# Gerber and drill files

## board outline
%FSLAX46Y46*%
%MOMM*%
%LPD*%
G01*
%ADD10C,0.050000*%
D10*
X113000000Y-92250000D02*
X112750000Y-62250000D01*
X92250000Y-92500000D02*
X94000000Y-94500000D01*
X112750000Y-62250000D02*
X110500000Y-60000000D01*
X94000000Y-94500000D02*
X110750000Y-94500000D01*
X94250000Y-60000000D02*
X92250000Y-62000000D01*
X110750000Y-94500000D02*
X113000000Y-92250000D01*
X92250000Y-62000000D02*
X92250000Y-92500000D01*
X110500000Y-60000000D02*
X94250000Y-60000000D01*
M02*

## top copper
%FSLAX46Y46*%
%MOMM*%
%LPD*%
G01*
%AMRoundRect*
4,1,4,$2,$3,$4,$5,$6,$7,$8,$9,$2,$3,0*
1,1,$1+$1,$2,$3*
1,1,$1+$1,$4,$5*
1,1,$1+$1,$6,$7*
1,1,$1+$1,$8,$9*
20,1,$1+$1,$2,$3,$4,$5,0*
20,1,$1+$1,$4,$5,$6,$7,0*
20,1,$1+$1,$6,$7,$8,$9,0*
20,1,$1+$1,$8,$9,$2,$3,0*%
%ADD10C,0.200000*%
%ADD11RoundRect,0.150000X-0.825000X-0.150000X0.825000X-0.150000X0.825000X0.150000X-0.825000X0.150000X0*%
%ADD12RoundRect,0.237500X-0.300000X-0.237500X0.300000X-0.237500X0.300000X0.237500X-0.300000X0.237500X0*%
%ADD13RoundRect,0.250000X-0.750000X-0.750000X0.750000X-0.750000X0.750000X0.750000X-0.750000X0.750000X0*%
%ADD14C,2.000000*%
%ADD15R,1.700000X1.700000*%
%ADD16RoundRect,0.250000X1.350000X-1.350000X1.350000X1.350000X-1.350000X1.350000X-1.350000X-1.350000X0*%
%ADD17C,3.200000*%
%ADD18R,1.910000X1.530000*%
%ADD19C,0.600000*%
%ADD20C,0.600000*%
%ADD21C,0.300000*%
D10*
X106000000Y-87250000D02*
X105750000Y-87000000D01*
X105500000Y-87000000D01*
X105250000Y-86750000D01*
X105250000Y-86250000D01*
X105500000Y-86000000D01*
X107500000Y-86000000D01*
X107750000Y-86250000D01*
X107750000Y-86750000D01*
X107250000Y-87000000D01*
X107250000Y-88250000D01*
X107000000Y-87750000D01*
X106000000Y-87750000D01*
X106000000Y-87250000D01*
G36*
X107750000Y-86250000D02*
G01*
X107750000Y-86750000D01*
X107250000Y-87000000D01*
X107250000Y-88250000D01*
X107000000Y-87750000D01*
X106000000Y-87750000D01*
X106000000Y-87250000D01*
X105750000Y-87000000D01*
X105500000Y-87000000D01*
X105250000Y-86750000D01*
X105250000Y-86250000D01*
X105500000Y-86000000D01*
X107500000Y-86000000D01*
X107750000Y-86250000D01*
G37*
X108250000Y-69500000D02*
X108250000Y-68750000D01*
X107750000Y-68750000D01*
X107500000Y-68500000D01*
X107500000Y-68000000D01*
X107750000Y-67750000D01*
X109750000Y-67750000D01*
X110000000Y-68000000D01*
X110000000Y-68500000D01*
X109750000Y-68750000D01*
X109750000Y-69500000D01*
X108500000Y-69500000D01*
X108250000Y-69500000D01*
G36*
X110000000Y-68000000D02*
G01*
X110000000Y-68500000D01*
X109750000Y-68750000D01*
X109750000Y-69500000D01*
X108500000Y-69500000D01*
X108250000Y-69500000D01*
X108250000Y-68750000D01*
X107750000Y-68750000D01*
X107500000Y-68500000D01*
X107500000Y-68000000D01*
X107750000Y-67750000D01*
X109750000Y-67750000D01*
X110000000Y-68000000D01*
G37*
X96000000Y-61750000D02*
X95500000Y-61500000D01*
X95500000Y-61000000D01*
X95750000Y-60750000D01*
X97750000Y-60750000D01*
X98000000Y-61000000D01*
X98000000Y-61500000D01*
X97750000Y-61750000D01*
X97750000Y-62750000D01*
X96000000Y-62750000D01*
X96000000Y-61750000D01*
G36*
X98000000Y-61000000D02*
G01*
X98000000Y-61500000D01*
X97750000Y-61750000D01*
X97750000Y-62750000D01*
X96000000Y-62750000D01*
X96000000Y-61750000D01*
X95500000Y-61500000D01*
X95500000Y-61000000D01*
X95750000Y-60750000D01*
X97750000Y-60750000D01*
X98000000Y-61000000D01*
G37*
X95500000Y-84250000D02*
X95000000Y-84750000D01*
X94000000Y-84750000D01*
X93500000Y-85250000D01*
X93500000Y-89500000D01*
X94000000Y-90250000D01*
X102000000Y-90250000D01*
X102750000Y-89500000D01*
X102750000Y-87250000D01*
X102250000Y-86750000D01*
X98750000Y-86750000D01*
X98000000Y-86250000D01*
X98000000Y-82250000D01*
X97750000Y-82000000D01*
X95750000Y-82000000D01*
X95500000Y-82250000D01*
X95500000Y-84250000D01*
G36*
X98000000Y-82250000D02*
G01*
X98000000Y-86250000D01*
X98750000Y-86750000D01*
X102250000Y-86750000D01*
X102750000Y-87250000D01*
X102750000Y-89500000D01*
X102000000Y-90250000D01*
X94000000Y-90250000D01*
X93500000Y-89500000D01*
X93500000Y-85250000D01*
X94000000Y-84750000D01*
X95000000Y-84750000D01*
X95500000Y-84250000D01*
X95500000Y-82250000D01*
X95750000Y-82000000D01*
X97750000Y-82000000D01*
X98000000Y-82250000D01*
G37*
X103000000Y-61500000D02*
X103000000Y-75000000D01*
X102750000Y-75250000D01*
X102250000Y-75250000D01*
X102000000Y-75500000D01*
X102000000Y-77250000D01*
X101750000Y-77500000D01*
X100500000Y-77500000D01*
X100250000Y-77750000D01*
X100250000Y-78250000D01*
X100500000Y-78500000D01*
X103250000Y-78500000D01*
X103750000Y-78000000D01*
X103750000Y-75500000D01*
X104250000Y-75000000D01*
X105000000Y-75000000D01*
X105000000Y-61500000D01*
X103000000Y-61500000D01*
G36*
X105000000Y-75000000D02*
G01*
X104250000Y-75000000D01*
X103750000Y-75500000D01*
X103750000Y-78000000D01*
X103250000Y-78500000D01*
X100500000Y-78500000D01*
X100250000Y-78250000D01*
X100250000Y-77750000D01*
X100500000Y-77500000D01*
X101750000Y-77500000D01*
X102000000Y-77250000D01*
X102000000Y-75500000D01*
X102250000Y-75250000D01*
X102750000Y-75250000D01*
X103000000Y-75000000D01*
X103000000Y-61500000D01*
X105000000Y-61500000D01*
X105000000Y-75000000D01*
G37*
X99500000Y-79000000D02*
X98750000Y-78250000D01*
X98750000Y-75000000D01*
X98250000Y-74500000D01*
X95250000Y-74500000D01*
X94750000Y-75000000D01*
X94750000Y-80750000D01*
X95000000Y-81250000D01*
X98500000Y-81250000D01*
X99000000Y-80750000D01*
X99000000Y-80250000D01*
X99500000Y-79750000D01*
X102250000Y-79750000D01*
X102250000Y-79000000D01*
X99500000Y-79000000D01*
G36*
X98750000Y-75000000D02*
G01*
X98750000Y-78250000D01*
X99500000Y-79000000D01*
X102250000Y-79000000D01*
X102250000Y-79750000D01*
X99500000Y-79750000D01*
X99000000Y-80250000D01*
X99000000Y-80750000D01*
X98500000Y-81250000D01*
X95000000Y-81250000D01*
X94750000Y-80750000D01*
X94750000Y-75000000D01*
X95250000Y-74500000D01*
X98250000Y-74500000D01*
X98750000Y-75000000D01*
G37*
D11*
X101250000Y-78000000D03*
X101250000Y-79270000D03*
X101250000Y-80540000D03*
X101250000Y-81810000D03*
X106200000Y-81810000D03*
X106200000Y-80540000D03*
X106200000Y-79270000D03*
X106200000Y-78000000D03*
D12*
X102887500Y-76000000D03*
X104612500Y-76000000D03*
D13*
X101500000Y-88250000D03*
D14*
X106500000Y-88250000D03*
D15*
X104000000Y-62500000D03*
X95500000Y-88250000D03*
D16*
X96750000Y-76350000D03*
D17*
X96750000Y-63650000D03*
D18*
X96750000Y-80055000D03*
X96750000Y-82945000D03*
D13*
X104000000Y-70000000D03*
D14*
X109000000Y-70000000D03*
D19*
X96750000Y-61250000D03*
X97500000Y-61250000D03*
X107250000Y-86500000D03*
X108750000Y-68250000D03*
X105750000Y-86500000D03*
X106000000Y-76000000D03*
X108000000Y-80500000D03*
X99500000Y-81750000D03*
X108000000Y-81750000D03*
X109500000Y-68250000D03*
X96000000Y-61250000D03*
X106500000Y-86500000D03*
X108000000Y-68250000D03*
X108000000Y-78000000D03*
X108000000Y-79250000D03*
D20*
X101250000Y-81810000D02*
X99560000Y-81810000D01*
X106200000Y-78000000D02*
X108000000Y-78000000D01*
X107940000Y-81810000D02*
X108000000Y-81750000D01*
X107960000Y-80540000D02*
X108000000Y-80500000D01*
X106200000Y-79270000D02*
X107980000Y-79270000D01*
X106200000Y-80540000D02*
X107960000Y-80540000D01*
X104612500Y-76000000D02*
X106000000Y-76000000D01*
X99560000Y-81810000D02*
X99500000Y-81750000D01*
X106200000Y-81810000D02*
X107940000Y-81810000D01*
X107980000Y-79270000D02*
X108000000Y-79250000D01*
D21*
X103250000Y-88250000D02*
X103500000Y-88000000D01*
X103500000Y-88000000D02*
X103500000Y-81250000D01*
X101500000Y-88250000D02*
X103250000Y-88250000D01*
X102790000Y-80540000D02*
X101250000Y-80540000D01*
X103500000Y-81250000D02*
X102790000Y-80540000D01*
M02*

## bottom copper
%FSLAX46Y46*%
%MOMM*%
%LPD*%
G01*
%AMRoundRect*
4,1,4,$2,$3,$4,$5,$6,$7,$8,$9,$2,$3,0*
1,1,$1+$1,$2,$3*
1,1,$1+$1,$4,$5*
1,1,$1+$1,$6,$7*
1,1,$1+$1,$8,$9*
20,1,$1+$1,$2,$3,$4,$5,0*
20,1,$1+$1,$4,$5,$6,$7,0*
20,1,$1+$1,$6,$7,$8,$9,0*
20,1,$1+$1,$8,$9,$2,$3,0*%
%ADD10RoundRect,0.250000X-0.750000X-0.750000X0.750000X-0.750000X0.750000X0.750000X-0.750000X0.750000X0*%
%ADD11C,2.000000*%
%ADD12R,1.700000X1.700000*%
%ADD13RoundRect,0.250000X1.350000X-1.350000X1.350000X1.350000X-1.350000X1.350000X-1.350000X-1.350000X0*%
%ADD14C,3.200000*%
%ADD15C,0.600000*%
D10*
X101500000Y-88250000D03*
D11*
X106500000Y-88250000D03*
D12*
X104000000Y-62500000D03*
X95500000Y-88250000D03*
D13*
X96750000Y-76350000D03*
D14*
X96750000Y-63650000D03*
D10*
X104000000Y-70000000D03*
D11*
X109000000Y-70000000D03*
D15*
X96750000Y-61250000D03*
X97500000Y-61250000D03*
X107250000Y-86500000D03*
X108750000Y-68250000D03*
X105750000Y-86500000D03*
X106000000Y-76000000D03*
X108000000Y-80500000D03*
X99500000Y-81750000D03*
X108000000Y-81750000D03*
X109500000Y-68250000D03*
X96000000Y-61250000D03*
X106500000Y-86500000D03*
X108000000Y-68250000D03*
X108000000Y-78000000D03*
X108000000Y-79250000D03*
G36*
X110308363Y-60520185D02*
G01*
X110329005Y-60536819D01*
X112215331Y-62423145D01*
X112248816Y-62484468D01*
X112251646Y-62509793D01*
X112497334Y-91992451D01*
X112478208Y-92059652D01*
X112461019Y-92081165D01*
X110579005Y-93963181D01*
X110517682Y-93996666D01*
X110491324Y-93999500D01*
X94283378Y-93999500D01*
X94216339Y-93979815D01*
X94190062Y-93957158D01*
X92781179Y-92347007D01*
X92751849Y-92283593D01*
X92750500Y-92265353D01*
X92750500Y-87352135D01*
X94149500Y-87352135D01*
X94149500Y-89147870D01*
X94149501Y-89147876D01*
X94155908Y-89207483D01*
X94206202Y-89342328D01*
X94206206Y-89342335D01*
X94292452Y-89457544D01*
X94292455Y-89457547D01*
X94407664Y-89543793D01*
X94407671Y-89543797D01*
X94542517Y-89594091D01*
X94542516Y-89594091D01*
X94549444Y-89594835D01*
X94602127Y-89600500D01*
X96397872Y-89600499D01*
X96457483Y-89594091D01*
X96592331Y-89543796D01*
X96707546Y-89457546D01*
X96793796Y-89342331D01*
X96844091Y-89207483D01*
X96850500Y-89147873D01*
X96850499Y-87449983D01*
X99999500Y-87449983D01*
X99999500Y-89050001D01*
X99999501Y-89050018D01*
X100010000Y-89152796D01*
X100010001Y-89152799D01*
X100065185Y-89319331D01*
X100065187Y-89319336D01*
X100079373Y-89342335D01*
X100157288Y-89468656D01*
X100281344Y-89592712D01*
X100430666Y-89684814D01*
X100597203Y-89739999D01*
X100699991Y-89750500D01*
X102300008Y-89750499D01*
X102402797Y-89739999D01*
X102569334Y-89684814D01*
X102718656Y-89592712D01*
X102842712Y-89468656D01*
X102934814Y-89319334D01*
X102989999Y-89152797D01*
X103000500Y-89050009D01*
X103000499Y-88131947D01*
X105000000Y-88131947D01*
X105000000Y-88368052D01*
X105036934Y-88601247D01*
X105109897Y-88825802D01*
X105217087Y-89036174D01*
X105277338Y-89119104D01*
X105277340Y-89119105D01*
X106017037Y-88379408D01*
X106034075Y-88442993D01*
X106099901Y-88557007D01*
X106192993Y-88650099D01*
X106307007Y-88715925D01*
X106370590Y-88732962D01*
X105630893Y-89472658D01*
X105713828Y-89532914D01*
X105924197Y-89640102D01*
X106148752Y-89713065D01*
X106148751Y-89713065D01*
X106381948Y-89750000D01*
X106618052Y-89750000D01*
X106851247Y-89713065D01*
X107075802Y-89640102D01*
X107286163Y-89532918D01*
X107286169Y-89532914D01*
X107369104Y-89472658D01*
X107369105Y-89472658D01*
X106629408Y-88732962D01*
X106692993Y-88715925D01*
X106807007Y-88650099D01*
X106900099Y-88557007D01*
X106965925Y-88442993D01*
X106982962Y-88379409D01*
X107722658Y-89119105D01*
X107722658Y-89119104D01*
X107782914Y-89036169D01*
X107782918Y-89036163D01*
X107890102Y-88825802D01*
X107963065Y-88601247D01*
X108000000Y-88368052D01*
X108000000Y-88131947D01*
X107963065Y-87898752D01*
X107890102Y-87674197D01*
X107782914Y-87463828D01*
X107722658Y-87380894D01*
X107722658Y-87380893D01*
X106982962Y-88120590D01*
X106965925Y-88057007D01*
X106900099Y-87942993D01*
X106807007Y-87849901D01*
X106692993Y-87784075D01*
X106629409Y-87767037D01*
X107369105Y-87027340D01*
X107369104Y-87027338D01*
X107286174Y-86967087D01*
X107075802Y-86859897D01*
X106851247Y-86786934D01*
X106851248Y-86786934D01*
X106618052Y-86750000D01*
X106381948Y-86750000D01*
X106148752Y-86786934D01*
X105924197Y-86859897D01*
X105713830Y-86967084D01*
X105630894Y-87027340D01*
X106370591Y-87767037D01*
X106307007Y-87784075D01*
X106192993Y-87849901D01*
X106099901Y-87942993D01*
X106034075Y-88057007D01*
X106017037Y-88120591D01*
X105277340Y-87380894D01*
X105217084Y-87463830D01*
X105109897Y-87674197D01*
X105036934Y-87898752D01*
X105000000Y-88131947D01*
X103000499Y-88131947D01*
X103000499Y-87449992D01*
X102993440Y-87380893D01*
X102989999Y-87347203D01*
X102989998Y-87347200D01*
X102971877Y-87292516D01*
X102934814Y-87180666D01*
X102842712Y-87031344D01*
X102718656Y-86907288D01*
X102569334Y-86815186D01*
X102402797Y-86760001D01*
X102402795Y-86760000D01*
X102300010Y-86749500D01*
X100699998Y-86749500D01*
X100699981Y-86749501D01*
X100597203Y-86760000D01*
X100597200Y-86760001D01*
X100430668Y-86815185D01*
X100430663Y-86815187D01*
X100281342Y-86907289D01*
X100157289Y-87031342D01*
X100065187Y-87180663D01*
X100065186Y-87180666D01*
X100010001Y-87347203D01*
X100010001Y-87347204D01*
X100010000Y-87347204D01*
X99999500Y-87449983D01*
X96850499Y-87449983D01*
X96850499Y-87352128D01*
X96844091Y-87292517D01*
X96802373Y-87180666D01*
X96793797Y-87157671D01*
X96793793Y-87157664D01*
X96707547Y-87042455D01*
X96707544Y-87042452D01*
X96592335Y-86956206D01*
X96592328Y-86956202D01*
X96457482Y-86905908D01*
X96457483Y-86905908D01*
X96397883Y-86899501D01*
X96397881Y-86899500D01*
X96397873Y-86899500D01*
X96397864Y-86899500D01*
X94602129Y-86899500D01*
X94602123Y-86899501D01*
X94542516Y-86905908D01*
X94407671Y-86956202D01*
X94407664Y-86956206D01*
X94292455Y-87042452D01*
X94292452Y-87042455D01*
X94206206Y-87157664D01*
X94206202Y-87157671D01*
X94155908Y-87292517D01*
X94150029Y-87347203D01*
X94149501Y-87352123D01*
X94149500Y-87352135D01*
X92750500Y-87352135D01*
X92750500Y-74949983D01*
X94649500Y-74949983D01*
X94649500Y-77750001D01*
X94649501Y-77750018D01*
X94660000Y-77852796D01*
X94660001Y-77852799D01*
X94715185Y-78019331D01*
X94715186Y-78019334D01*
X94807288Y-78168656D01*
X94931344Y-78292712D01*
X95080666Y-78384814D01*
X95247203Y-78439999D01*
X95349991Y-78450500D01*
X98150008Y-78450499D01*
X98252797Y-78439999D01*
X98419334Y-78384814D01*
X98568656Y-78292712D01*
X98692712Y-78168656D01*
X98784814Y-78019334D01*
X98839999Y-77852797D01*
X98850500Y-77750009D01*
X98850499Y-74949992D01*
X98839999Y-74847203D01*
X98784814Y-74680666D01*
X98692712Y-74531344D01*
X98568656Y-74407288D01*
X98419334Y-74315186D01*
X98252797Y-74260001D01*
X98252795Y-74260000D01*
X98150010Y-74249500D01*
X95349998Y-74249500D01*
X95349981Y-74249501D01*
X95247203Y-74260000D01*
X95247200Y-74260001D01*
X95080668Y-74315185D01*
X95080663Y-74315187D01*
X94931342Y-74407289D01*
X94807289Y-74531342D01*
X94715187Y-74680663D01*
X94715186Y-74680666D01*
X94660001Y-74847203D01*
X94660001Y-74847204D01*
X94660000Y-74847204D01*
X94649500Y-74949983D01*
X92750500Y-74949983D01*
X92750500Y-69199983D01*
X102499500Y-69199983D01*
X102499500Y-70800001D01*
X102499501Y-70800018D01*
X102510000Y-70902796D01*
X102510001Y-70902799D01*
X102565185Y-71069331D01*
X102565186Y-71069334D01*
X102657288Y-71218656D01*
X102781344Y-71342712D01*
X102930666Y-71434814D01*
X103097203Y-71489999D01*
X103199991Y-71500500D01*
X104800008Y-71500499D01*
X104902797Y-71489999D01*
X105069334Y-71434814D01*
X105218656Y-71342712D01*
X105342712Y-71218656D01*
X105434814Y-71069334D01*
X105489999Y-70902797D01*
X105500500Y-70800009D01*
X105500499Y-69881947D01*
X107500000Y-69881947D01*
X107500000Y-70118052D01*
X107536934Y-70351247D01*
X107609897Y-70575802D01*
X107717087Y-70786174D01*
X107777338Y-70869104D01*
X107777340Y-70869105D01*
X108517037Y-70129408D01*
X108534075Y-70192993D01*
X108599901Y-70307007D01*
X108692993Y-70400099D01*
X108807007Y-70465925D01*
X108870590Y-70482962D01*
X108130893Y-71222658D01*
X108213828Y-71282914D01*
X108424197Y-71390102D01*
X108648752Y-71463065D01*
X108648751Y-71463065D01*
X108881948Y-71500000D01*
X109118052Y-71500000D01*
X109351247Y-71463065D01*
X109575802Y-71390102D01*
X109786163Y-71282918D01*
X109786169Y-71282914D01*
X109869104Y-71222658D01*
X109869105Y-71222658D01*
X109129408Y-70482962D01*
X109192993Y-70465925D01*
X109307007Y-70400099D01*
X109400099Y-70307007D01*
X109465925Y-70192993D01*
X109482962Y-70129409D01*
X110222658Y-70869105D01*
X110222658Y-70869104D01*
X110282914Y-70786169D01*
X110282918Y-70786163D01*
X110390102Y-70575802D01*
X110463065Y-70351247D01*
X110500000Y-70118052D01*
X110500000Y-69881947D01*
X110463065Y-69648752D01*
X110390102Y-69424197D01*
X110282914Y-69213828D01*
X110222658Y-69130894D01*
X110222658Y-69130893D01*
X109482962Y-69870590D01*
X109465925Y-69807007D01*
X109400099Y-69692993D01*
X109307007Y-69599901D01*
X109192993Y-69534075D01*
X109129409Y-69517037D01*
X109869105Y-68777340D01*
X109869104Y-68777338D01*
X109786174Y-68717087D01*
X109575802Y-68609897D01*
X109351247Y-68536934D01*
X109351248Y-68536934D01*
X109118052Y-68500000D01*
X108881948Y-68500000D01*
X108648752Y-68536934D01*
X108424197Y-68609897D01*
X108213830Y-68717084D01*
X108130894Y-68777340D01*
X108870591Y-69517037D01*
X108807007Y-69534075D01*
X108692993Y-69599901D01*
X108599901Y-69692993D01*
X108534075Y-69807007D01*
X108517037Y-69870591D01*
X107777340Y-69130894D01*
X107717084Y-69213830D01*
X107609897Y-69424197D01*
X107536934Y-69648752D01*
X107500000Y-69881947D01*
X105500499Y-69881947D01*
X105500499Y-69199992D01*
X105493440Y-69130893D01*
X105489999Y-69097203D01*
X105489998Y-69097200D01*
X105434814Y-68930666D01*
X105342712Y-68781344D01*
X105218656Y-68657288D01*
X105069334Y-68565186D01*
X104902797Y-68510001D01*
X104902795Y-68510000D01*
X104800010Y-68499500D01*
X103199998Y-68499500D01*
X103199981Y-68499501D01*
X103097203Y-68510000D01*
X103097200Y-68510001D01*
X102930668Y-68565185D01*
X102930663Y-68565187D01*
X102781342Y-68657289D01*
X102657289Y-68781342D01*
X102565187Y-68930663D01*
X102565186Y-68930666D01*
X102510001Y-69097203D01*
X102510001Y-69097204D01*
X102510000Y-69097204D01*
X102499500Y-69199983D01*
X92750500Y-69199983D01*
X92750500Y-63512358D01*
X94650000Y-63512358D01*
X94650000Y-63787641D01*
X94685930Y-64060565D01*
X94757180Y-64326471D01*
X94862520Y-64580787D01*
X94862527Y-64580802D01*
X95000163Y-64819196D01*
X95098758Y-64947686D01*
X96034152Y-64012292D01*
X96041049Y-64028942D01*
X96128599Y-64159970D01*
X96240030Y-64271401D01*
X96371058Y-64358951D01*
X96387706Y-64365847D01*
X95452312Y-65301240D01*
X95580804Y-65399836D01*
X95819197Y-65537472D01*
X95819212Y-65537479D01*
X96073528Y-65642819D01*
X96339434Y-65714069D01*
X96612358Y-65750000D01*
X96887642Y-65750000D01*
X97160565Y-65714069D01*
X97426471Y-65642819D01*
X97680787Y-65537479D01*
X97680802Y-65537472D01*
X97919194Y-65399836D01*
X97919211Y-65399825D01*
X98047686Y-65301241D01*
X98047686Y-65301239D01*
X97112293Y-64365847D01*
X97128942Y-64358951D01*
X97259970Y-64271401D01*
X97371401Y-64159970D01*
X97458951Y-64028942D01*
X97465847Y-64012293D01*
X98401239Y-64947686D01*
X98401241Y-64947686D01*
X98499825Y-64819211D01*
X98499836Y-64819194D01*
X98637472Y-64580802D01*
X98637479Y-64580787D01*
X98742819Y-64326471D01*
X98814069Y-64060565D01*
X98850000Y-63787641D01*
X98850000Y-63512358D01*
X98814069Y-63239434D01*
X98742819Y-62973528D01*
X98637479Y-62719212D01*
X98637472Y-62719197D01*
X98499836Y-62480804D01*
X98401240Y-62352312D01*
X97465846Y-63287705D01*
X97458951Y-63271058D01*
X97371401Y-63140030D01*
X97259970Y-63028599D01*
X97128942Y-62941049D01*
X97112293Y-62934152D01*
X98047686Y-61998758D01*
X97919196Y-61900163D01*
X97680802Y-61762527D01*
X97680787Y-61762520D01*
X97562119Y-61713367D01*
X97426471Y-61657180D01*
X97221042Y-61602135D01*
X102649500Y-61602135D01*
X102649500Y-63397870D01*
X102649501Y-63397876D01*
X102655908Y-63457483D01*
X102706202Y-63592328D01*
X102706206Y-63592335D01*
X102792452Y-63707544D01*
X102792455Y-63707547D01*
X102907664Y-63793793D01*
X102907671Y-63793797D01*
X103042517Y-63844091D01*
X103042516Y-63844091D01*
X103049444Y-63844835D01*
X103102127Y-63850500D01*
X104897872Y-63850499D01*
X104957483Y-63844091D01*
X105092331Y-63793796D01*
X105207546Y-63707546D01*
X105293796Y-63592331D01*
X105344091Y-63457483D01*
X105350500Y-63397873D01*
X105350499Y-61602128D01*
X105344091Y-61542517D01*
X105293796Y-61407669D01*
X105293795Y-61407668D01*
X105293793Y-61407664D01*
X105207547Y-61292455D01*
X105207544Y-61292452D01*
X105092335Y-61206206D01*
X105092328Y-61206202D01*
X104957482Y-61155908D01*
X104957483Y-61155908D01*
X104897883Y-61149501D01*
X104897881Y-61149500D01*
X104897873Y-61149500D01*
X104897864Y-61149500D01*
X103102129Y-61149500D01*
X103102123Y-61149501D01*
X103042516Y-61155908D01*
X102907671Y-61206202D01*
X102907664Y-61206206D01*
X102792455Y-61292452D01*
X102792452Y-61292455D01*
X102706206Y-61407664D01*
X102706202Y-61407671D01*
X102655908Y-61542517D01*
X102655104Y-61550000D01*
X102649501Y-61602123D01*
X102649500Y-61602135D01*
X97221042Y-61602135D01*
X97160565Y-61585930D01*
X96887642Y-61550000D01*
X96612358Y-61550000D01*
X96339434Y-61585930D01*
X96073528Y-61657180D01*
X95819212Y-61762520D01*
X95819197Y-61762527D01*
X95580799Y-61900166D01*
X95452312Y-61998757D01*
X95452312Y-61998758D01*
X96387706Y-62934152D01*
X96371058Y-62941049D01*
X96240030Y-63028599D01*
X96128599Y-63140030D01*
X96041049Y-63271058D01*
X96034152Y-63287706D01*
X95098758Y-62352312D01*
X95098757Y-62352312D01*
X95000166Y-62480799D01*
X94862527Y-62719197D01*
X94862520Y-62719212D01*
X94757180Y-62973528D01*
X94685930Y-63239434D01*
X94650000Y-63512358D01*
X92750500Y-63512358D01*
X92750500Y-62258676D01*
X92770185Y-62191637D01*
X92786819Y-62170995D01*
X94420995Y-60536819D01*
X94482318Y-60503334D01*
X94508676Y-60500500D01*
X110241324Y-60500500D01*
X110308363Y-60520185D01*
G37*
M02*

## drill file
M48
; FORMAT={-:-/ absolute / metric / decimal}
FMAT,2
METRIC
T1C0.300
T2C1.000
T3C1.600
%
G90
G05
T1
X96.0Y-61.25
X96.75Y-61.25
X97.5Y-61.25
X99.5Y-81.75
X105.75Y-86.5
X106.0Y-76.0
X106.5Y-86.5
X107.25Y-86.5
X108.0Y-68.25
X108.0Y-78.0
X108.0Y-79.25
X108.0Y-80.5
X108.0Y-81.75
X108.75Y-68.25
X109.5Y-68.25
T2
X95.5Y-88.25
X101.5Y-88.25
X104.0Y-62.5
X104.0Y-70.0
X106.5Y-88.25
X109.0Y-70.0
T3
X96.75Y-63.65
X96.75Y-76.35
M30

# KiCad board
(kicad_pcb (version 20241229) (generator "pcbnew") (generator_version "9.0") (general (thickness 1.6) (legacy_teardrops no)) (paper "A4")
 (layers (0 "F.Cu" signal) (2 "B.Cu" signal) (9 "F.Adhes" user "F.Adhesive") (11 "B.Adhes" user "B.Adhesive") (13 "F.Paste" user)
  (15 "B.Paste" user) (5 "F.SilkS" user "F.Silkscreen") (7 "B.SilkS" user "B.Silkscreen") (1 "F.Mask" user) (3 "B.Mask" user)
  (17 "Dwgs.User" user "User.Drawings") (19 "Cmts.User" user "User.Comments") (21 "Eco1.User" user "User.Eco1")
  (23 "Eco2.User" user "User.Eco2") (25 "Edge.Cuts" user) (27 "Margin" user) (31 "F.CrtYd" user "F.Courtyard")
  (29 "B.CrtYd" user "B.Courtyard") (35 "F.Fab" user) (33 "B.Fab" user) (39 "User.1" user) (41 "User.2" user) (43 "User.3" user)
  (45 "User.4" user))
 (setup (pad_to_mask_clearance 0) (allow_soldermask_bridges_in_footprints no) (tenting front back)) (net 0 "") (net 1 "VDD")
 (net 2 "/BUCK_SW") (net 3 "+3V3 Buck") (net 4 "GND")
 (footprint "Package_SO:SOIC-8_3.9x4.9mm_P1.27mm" (layer "F.Cu") (at 103.725 79.905)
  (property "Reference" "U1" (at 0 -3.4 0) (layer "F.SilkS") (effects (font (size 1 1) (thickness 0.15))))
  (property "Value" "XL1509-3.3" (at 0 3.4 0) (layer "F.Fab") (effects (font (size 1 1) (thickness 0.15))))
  (pad "1" smd roundrect (at -2.475 -1.905) (size 1.95 0.6) (layers "F.Cu" "F.Mask" "F.Paste") (roundrect_rratio 0.25) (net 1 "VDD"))
  (pad "2" smd roundrect (at -2.475 -0.635) (size 1.95 0.6) (layers "F.Cu" "F.Mask" "F.Paste") (roundrect_rratio 0.25) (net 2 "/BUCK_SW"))
  (pad "3" smd roundrect (at -2.475 0.635) (size 1.95 0.6) (layers "F.Cu" "F.Mask" "F.Paste") (roundrect_rratio 0.25) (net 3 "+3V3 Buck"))
  (pad "4" smd roundrect (at -2.475 1.905) (size 1.95 0.6) (layers "F.Cu" "F.Mask" "F.Paste") (roundrect_rratio 0.25) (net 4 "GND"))
  (pad "5" smd roundrect (at 2.475 1.905) (size 1.95 0.6) (layers "F.Cu" "F.Mask" "F.Paste") (roundrect_rratio 0.25) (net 4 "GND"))
  (pad "6" smd roundrect (at 2.475 0.635) (size 1.95 0.6) (layers "F.Cu" "F.Mask" "F.Paste") (roundrect_rratio 0.25) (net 4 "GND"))
  (pad "7" smd roundrect (at 2.475 -0.635) (size 1.95 0.6) (layers "F.Cu" "F.Mask" "F.Paste") (roundrect_rratio 0.25) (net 4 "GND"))
  (pad "8" smd roundrect (at 2.475 -1.905) (size 1.95 0.6) (layers "F.Cu" "F.Mask" "F.Paste") (roundrect_rratio 0.25) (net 4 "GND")))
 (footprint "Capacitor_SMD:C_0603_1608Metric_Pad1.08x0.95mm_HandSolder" (layer "F.Cu") (at 103.75 76)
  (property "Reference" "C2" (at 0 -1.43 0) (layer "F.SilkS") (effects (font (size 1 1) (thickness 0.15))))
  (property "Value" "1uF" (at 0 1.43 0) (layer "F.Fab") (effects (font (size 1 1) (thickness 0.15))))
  (pad "1" smd roundrect (at -0.8625 0) (size 1.075 0.95) (layers "F.Cu" "F.Mask" "F.Paste") (roundrect_rratio 0.25) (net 1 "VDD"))
  (pad "2" smd roundrect (at 0.8625 0) (size 1.075 0.95) (layers "F.Cu" "F.Mask" "F.Paste") (roundrect_rratio 0.25) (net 4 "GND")))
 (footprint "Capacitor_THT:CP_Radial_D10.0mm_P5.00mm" (layer "F.Cu") (at 101.5 88.25)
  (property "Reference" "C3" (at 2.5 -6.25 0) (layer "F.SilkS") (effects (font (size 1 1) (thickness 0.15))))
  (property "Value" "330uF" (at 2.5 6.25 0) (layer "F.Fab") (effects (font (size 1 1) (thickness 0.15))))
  (pad "1" thru_hole roundrect (at 0 0) (size 2 2) (drill 1) (layers "*.Cu" "*.Mask") (remove_unused_layers no) (roundrect_rratio 0.125)
   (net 3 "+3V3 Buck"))
  (pad "2" thru_hole circle (at 5 0) (size 2 2) (drill 1) (layers "*.Cu" "*.Mask") (remove_unused_layers no) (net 4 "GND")))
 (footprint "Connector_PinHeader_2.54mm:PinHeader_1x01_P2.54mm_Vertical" (layer "F.Cu") (at 104 62.5)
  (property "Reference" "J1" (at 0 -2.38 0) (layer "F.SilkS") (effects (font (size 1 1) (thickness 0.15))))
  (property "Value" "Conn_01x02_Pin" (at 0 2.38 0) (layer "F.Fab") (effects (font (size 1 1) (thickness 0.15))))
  (pad "1" thru_hole rect (at 0 0) (size 1.7 1.7) (drill 1) (layers "*.Cu" "*.Mask") (remove_unused_layers no) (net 1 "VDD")))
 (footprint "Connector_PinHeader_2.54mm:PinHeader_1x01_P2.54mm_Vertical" (layer "F.Cu") (at 95.5 88.25)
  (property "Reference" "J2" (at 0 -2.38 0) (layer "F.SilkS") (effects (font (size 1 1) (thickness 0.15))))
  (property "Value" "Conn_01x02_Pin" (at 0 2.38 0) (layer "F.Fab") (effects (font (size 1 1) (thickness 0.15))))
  (pad "1" thru_hole rect (at 0 0) (size 1.7 1.7) (drill 1) (layers "*.Cu" "*.Mask") (remove_unused_layers no) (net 3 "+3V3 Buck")))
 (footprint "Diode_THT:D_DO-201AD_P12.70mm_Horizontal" (layer "F.Cu") (at 96.75 76.35 90)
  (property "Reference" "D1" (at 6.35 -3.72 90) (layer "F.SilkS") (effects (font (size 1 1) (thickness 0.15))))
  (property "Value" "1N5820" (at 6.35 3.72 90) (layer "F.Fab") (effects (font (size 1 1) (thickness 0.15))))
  (pad "1" thru_hole roundrect (at 0 0 90) (size 3.2 3.2) (drill 1.6) (layers "*.Cu" "*.Mask") (remove_unused_layers no)
   (roundrect_rratio 0.078125) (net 2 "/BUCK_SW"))
  (pad "2" thru_hole circle (at 12.7 0 90) (size 3.2 3.2) (drill 1.6) (layers "*.Cu" "*.Mask") (remove_unused_layers no) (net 4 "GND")))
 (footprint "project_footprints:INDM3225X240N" (layer "F.Cu") (at 96.75 81.5 -90)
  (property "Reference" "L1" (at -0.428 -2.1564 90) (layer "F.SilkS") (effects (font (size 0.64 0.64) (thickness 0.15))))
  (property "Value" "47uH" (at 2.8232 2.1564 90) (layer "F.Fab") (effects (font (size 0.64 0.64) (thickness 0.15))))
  (pad "1" smd rect (at -1.445 0 270) (size 1.53 1.91) (layers "F.Cu" "F.Mask" "F.Paste") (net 2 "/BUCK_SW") (solder_mask_margin 0.102))
  (pad "2" smd rect (at 1.445 0 270) (size 1.53 1.91) (layers "F.Cu" "F.Mask" "F.Paste") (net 3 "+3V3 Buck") (solder_mask_margin 0.102)))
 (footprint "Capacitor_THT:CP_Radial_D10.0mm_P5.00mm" (layer "F.Cu") (at 104 70)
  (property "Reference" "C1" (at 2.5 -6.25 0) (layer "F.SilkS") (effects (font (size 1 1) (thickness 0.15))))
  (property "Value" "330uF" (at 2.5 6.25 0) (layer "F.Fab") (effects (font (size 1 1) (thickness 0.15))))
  (pad "1" thru_hole roundrect (at 0 0) (size 2 2) (drill 1) (layers "*.Cu" "*.Mask") (remove_unused_layers no) (roundrect_rratio 0.125)
   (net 1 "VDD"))
  (pad "2" thru_hole circle (at 5 0) (size 2 2) (drill 1) (layers "*.Cu" "*.Mask") (remove_unused_layers no) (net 4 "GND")))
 (gr_poly
  (pts (xy 106 87.25) (xy 105.75 87) (xy 105.5 87) (xy 105.25 86.75) (xy 105.25 86.25) (xy 105.5 86) (xy 107.5 86) (xy 107.75 86.25)
   (xy 107.75 86.75) (xy 107.25 87) (xy 107.25 88.25) (xy 107.25 88.25) (xy 107 87.75) (xy 106 87.75))
  (stroke (width 0.2) (type solid)) (fill yes) (layer "F.Cu") (net 4))
 (gr_poly
  (pts (xy 108.25 69.5) (xy 108.25 68.75) (xy 107.75 68.75) (xy 107.5 68.5) (xy 107.5 68) (xy 107.75 67.75) (xy 109.75 67.75) (xy 110 68)
   (xy 110 68.5) (xy 109.75 68.75) (xy 109.75 69.5) (xy 108.5 69.5))
  (stroke (width 0.2) (type solid)) (fill yes) (layer "F.Cu") (net 4))
 (gr_poly
  (pts (xy 96 61.75) (xy 95.5 61.5) (xy 95.5 61) (xy 95.75 60.75) (xy 97.75 60.75) (xy 98 61) (xy 98 61.5) (xy 97.75 61.75) (xy 97.75 62.75)
   (xy 96 62.75))
  (stroke (width 0.2) (type solid)) (fill yes) (layer "F.Cu") (net 4))
 (gr_poly
  (pts (xy 95.5 84.25) (xy 95 84.75) (xy 94 84.75) (xy 93.5 85.25) (xy 93.5 89.5) (xy 94 90.25) (xy 102 90.25) (xy 102.75 89.5)
   (xy 102.75 87.25) (xy 102.25 86.75) (xy 98.75 86.75) (xy 98 86.25) (xy 98 82.25) (xy 97.75 82) (xy 95.75 82) (xy 95.5 82.25))
  (stroke (width 0.2) (type solid)) (fill yes) (layer "F.Cu") (net 3))
 (gr_poly
  (pts (xy 103 61.5) (xy 103 75) (xy 102.75 75.25) (xy 102.25 75.25) (xy 102 75.5) (xy 102 77.25) (xy 101.75 77.5) (xy 100.5 77.5)
   (xy 100.25 77.75) (xy 100.25 78.25) (xy 100.5 78.5) (xy 103.25 78.5) (xy 103.75 78) (xy 103.75 75.5) (xy 104.25 75) (xy 105 75)
   (xy 105 61.5))
  (stroke (width 0.2) (type solid)) (fill yes) (layer "F.Cu") (net 1))
 (gr_poly
  (pts (xy 99.5 79) (xy 98.75 78.25) (xy 98.75 75) (xy 98.25 74.5) (xy 95.25 74.5) (xy 94.75 75) (xy 94.75 80.75) (xy 95 81.25)
   (xy 98.5 81.25) (xy 99 80.75) (xy 99 80.25) (xy 99.5 79.75) (xy 102.25 79.75) (xy 102.25 79))
  (stroke (width 0.2) (type solid)) (fill yes) (layer "F.Cu") (net 2))
 (gr_line (start 113 92.25) (end 112.75 62.25) (stroke (width 0.05) (type default)) (layer "Edge.Cuts"))
 (gr_line (start 92.25 92.5) (end 94 94.5) (stroke (width 0.05) (type default)) (layer "Edge.Cuts"))
 (gr_line (start 112.75 62.25) (end 110.5 60) (stroke (width 0.05) (type default)) (layer "Edge.Cuts"))
 (gr_line (start 94 94.5) (end 110.75 94.5) (stroke (width 0.05) (type default)) (layer "Edge.Cuts"))
 (gr_line (start 94.25 60) (end 92.25 62) (stroke (width 0.05) (type default)) (layer "Edge.Cuts"))
 (gr_line (start 110.75 94.5) (end 113 92.25) (stroke (width 0.05) (type default)) (layer "Edge.Cuts"))
 (gr_line (start 92.25 62) (end 92.25 92.5) (stroke (width 0.05) (type default)) (layer "Edge.Cuts"))
 (gr_line (start 110.5 60) (end 94.25 60) (stroke (width 0.05) (type default)) (layer "Edge.Cuts"))
 (segment (start 101.25 81.81) (end 99.56 81.81) (width 0.6) (layer "F.Cu") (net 4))
 (segment (start 106.2 78) (end 108 78) (width 0.6) (layer "F.Cu") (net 4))
 (segment (start 107.94 81.81) (end 108 81.75) (width 0.6) (layer "F.Cu") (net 4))
 (segment (start 107.96 80.54) (end 108 80.5) (width 0.6) (layer "F.Cu") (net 4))
 (segment (start 106.2 79.27) (end 107.98 79.27) (width 0.6) (layer "F.Cu") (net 4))
 (segment (start 106.2 80.54) (end 107.96 80.54) (width 0.6) (layer "F.Cu") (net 4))
 (segment (start 104.6125 76) (end 106 76) (width 0.6) (layer "F.Cu") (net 4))
 (segment (start 99.56 81.81) (end 99.5 81.75) (width 0.6) (layer "F.Cu") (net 4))
 (segment (start 106.2 81.81) (end 107.94 81.81) (width 0.6) (layer "F.Cu") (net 4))
 (segment (start 107.98 79.27) (end 108 79.25) (width 0.6) (layer "F.Cu") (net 4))
 (via (at 96.75 61.25) (size 0.6) (drill 0.3) (layers "F.Cu" "B.Cu") (free yes) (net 4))
 (via (at 97.5 61.25) (size 0.6) (drill 0.3) (layers "F.Cu" "B.Cu") (free yes) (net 4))
 (via (at 107.25 86.5) (size 0.6) (drill 0.3) (layers "F.Cu" "B.Cu") (free yes) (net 4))
 (via (at 108.75 68.25) (size 0.6) (drill 0.3) (layers "F.Cu" "B.Cu") (free yes) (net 4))
 (via (at 105.75 86.5) (size 0.6) (drill 0.3) (layers "F.Cu" "B.Cu") (free yes) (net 4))
 (via (at 106 76) (size 0.6) (drill 0.3) (layers "F.Cu" "B.Cu") (free yes) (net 4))
 (via (at 108 80.5) (size 0.6) (drill 0.3) (layers "F.Cu" "B.Cu") (free yes) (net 4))
 (via (at 99.5 81.75) (size 0.6) (drill 0.3) (layers "F.Cu" "B.Cu") (free yes) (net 4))
 (via (at 108 81.75) (size 0.6) (drill 0.3) (layers "F.Cu" "B.Cu") (free yes) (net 4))
 (via (at 109.5 68.25) (size 0.6) (drill 0.3) (layers "F.Cu" "B.Cu") (free yes) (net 4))
 (via (at 96 61.25) (size 0.6) (drill 0.3) (layers "F.Cu" "B.Cu") (free yes) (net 4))
 (via (at 106.5 86.5) (size 0.6) (drill 0.3) (layers "F.Cu" "B.Cu") (free yes) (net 4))
 (via (at 108 68.25) (size 0.6) (drill 0.3) (layers "F.Cu" "B.Cu") (free yes) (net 4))
 (via (at 108 78) (size 0.6) (drill 0.3) (layers "F.Cu" "B.Cu") (free yes) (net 4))
 (via (at 108 79.25) (size 0.6) (drill 0.3) (layers "F.Cu" "B.Cu") (free yes) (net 4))
 (segment (start 103.25 88.25) (end 103.5 88) (width 0.3) (layer "F.Cu") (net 3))
 (segment (start 103.5 88) (end 103.5 81.25) (width 0.3) (layer "F.Cu") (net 3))
 (segment (start 101.5 88.25) (end 103.25 88.25) (width 0.3) (layer "F.Cu") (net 3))
 (segment (start 102.79 80.54) (end 101.25 80.54) (width 0.3) (layer "F.Cu") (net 3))
 (segment (start 103.5 81.25) (end 102.79 80.54) (width 0.3) (layer "F.Cu") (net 3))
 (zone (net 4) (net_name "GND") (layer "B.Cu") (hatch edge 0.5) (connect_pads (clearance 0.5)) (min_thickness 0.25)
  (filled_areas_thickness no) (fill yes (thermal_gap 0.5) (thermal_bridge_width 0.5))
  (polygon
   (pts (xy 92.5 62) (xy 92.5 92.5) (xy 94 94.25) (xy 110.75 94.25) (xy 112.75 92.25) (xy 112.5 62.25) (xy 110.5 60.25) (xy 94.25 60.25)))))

